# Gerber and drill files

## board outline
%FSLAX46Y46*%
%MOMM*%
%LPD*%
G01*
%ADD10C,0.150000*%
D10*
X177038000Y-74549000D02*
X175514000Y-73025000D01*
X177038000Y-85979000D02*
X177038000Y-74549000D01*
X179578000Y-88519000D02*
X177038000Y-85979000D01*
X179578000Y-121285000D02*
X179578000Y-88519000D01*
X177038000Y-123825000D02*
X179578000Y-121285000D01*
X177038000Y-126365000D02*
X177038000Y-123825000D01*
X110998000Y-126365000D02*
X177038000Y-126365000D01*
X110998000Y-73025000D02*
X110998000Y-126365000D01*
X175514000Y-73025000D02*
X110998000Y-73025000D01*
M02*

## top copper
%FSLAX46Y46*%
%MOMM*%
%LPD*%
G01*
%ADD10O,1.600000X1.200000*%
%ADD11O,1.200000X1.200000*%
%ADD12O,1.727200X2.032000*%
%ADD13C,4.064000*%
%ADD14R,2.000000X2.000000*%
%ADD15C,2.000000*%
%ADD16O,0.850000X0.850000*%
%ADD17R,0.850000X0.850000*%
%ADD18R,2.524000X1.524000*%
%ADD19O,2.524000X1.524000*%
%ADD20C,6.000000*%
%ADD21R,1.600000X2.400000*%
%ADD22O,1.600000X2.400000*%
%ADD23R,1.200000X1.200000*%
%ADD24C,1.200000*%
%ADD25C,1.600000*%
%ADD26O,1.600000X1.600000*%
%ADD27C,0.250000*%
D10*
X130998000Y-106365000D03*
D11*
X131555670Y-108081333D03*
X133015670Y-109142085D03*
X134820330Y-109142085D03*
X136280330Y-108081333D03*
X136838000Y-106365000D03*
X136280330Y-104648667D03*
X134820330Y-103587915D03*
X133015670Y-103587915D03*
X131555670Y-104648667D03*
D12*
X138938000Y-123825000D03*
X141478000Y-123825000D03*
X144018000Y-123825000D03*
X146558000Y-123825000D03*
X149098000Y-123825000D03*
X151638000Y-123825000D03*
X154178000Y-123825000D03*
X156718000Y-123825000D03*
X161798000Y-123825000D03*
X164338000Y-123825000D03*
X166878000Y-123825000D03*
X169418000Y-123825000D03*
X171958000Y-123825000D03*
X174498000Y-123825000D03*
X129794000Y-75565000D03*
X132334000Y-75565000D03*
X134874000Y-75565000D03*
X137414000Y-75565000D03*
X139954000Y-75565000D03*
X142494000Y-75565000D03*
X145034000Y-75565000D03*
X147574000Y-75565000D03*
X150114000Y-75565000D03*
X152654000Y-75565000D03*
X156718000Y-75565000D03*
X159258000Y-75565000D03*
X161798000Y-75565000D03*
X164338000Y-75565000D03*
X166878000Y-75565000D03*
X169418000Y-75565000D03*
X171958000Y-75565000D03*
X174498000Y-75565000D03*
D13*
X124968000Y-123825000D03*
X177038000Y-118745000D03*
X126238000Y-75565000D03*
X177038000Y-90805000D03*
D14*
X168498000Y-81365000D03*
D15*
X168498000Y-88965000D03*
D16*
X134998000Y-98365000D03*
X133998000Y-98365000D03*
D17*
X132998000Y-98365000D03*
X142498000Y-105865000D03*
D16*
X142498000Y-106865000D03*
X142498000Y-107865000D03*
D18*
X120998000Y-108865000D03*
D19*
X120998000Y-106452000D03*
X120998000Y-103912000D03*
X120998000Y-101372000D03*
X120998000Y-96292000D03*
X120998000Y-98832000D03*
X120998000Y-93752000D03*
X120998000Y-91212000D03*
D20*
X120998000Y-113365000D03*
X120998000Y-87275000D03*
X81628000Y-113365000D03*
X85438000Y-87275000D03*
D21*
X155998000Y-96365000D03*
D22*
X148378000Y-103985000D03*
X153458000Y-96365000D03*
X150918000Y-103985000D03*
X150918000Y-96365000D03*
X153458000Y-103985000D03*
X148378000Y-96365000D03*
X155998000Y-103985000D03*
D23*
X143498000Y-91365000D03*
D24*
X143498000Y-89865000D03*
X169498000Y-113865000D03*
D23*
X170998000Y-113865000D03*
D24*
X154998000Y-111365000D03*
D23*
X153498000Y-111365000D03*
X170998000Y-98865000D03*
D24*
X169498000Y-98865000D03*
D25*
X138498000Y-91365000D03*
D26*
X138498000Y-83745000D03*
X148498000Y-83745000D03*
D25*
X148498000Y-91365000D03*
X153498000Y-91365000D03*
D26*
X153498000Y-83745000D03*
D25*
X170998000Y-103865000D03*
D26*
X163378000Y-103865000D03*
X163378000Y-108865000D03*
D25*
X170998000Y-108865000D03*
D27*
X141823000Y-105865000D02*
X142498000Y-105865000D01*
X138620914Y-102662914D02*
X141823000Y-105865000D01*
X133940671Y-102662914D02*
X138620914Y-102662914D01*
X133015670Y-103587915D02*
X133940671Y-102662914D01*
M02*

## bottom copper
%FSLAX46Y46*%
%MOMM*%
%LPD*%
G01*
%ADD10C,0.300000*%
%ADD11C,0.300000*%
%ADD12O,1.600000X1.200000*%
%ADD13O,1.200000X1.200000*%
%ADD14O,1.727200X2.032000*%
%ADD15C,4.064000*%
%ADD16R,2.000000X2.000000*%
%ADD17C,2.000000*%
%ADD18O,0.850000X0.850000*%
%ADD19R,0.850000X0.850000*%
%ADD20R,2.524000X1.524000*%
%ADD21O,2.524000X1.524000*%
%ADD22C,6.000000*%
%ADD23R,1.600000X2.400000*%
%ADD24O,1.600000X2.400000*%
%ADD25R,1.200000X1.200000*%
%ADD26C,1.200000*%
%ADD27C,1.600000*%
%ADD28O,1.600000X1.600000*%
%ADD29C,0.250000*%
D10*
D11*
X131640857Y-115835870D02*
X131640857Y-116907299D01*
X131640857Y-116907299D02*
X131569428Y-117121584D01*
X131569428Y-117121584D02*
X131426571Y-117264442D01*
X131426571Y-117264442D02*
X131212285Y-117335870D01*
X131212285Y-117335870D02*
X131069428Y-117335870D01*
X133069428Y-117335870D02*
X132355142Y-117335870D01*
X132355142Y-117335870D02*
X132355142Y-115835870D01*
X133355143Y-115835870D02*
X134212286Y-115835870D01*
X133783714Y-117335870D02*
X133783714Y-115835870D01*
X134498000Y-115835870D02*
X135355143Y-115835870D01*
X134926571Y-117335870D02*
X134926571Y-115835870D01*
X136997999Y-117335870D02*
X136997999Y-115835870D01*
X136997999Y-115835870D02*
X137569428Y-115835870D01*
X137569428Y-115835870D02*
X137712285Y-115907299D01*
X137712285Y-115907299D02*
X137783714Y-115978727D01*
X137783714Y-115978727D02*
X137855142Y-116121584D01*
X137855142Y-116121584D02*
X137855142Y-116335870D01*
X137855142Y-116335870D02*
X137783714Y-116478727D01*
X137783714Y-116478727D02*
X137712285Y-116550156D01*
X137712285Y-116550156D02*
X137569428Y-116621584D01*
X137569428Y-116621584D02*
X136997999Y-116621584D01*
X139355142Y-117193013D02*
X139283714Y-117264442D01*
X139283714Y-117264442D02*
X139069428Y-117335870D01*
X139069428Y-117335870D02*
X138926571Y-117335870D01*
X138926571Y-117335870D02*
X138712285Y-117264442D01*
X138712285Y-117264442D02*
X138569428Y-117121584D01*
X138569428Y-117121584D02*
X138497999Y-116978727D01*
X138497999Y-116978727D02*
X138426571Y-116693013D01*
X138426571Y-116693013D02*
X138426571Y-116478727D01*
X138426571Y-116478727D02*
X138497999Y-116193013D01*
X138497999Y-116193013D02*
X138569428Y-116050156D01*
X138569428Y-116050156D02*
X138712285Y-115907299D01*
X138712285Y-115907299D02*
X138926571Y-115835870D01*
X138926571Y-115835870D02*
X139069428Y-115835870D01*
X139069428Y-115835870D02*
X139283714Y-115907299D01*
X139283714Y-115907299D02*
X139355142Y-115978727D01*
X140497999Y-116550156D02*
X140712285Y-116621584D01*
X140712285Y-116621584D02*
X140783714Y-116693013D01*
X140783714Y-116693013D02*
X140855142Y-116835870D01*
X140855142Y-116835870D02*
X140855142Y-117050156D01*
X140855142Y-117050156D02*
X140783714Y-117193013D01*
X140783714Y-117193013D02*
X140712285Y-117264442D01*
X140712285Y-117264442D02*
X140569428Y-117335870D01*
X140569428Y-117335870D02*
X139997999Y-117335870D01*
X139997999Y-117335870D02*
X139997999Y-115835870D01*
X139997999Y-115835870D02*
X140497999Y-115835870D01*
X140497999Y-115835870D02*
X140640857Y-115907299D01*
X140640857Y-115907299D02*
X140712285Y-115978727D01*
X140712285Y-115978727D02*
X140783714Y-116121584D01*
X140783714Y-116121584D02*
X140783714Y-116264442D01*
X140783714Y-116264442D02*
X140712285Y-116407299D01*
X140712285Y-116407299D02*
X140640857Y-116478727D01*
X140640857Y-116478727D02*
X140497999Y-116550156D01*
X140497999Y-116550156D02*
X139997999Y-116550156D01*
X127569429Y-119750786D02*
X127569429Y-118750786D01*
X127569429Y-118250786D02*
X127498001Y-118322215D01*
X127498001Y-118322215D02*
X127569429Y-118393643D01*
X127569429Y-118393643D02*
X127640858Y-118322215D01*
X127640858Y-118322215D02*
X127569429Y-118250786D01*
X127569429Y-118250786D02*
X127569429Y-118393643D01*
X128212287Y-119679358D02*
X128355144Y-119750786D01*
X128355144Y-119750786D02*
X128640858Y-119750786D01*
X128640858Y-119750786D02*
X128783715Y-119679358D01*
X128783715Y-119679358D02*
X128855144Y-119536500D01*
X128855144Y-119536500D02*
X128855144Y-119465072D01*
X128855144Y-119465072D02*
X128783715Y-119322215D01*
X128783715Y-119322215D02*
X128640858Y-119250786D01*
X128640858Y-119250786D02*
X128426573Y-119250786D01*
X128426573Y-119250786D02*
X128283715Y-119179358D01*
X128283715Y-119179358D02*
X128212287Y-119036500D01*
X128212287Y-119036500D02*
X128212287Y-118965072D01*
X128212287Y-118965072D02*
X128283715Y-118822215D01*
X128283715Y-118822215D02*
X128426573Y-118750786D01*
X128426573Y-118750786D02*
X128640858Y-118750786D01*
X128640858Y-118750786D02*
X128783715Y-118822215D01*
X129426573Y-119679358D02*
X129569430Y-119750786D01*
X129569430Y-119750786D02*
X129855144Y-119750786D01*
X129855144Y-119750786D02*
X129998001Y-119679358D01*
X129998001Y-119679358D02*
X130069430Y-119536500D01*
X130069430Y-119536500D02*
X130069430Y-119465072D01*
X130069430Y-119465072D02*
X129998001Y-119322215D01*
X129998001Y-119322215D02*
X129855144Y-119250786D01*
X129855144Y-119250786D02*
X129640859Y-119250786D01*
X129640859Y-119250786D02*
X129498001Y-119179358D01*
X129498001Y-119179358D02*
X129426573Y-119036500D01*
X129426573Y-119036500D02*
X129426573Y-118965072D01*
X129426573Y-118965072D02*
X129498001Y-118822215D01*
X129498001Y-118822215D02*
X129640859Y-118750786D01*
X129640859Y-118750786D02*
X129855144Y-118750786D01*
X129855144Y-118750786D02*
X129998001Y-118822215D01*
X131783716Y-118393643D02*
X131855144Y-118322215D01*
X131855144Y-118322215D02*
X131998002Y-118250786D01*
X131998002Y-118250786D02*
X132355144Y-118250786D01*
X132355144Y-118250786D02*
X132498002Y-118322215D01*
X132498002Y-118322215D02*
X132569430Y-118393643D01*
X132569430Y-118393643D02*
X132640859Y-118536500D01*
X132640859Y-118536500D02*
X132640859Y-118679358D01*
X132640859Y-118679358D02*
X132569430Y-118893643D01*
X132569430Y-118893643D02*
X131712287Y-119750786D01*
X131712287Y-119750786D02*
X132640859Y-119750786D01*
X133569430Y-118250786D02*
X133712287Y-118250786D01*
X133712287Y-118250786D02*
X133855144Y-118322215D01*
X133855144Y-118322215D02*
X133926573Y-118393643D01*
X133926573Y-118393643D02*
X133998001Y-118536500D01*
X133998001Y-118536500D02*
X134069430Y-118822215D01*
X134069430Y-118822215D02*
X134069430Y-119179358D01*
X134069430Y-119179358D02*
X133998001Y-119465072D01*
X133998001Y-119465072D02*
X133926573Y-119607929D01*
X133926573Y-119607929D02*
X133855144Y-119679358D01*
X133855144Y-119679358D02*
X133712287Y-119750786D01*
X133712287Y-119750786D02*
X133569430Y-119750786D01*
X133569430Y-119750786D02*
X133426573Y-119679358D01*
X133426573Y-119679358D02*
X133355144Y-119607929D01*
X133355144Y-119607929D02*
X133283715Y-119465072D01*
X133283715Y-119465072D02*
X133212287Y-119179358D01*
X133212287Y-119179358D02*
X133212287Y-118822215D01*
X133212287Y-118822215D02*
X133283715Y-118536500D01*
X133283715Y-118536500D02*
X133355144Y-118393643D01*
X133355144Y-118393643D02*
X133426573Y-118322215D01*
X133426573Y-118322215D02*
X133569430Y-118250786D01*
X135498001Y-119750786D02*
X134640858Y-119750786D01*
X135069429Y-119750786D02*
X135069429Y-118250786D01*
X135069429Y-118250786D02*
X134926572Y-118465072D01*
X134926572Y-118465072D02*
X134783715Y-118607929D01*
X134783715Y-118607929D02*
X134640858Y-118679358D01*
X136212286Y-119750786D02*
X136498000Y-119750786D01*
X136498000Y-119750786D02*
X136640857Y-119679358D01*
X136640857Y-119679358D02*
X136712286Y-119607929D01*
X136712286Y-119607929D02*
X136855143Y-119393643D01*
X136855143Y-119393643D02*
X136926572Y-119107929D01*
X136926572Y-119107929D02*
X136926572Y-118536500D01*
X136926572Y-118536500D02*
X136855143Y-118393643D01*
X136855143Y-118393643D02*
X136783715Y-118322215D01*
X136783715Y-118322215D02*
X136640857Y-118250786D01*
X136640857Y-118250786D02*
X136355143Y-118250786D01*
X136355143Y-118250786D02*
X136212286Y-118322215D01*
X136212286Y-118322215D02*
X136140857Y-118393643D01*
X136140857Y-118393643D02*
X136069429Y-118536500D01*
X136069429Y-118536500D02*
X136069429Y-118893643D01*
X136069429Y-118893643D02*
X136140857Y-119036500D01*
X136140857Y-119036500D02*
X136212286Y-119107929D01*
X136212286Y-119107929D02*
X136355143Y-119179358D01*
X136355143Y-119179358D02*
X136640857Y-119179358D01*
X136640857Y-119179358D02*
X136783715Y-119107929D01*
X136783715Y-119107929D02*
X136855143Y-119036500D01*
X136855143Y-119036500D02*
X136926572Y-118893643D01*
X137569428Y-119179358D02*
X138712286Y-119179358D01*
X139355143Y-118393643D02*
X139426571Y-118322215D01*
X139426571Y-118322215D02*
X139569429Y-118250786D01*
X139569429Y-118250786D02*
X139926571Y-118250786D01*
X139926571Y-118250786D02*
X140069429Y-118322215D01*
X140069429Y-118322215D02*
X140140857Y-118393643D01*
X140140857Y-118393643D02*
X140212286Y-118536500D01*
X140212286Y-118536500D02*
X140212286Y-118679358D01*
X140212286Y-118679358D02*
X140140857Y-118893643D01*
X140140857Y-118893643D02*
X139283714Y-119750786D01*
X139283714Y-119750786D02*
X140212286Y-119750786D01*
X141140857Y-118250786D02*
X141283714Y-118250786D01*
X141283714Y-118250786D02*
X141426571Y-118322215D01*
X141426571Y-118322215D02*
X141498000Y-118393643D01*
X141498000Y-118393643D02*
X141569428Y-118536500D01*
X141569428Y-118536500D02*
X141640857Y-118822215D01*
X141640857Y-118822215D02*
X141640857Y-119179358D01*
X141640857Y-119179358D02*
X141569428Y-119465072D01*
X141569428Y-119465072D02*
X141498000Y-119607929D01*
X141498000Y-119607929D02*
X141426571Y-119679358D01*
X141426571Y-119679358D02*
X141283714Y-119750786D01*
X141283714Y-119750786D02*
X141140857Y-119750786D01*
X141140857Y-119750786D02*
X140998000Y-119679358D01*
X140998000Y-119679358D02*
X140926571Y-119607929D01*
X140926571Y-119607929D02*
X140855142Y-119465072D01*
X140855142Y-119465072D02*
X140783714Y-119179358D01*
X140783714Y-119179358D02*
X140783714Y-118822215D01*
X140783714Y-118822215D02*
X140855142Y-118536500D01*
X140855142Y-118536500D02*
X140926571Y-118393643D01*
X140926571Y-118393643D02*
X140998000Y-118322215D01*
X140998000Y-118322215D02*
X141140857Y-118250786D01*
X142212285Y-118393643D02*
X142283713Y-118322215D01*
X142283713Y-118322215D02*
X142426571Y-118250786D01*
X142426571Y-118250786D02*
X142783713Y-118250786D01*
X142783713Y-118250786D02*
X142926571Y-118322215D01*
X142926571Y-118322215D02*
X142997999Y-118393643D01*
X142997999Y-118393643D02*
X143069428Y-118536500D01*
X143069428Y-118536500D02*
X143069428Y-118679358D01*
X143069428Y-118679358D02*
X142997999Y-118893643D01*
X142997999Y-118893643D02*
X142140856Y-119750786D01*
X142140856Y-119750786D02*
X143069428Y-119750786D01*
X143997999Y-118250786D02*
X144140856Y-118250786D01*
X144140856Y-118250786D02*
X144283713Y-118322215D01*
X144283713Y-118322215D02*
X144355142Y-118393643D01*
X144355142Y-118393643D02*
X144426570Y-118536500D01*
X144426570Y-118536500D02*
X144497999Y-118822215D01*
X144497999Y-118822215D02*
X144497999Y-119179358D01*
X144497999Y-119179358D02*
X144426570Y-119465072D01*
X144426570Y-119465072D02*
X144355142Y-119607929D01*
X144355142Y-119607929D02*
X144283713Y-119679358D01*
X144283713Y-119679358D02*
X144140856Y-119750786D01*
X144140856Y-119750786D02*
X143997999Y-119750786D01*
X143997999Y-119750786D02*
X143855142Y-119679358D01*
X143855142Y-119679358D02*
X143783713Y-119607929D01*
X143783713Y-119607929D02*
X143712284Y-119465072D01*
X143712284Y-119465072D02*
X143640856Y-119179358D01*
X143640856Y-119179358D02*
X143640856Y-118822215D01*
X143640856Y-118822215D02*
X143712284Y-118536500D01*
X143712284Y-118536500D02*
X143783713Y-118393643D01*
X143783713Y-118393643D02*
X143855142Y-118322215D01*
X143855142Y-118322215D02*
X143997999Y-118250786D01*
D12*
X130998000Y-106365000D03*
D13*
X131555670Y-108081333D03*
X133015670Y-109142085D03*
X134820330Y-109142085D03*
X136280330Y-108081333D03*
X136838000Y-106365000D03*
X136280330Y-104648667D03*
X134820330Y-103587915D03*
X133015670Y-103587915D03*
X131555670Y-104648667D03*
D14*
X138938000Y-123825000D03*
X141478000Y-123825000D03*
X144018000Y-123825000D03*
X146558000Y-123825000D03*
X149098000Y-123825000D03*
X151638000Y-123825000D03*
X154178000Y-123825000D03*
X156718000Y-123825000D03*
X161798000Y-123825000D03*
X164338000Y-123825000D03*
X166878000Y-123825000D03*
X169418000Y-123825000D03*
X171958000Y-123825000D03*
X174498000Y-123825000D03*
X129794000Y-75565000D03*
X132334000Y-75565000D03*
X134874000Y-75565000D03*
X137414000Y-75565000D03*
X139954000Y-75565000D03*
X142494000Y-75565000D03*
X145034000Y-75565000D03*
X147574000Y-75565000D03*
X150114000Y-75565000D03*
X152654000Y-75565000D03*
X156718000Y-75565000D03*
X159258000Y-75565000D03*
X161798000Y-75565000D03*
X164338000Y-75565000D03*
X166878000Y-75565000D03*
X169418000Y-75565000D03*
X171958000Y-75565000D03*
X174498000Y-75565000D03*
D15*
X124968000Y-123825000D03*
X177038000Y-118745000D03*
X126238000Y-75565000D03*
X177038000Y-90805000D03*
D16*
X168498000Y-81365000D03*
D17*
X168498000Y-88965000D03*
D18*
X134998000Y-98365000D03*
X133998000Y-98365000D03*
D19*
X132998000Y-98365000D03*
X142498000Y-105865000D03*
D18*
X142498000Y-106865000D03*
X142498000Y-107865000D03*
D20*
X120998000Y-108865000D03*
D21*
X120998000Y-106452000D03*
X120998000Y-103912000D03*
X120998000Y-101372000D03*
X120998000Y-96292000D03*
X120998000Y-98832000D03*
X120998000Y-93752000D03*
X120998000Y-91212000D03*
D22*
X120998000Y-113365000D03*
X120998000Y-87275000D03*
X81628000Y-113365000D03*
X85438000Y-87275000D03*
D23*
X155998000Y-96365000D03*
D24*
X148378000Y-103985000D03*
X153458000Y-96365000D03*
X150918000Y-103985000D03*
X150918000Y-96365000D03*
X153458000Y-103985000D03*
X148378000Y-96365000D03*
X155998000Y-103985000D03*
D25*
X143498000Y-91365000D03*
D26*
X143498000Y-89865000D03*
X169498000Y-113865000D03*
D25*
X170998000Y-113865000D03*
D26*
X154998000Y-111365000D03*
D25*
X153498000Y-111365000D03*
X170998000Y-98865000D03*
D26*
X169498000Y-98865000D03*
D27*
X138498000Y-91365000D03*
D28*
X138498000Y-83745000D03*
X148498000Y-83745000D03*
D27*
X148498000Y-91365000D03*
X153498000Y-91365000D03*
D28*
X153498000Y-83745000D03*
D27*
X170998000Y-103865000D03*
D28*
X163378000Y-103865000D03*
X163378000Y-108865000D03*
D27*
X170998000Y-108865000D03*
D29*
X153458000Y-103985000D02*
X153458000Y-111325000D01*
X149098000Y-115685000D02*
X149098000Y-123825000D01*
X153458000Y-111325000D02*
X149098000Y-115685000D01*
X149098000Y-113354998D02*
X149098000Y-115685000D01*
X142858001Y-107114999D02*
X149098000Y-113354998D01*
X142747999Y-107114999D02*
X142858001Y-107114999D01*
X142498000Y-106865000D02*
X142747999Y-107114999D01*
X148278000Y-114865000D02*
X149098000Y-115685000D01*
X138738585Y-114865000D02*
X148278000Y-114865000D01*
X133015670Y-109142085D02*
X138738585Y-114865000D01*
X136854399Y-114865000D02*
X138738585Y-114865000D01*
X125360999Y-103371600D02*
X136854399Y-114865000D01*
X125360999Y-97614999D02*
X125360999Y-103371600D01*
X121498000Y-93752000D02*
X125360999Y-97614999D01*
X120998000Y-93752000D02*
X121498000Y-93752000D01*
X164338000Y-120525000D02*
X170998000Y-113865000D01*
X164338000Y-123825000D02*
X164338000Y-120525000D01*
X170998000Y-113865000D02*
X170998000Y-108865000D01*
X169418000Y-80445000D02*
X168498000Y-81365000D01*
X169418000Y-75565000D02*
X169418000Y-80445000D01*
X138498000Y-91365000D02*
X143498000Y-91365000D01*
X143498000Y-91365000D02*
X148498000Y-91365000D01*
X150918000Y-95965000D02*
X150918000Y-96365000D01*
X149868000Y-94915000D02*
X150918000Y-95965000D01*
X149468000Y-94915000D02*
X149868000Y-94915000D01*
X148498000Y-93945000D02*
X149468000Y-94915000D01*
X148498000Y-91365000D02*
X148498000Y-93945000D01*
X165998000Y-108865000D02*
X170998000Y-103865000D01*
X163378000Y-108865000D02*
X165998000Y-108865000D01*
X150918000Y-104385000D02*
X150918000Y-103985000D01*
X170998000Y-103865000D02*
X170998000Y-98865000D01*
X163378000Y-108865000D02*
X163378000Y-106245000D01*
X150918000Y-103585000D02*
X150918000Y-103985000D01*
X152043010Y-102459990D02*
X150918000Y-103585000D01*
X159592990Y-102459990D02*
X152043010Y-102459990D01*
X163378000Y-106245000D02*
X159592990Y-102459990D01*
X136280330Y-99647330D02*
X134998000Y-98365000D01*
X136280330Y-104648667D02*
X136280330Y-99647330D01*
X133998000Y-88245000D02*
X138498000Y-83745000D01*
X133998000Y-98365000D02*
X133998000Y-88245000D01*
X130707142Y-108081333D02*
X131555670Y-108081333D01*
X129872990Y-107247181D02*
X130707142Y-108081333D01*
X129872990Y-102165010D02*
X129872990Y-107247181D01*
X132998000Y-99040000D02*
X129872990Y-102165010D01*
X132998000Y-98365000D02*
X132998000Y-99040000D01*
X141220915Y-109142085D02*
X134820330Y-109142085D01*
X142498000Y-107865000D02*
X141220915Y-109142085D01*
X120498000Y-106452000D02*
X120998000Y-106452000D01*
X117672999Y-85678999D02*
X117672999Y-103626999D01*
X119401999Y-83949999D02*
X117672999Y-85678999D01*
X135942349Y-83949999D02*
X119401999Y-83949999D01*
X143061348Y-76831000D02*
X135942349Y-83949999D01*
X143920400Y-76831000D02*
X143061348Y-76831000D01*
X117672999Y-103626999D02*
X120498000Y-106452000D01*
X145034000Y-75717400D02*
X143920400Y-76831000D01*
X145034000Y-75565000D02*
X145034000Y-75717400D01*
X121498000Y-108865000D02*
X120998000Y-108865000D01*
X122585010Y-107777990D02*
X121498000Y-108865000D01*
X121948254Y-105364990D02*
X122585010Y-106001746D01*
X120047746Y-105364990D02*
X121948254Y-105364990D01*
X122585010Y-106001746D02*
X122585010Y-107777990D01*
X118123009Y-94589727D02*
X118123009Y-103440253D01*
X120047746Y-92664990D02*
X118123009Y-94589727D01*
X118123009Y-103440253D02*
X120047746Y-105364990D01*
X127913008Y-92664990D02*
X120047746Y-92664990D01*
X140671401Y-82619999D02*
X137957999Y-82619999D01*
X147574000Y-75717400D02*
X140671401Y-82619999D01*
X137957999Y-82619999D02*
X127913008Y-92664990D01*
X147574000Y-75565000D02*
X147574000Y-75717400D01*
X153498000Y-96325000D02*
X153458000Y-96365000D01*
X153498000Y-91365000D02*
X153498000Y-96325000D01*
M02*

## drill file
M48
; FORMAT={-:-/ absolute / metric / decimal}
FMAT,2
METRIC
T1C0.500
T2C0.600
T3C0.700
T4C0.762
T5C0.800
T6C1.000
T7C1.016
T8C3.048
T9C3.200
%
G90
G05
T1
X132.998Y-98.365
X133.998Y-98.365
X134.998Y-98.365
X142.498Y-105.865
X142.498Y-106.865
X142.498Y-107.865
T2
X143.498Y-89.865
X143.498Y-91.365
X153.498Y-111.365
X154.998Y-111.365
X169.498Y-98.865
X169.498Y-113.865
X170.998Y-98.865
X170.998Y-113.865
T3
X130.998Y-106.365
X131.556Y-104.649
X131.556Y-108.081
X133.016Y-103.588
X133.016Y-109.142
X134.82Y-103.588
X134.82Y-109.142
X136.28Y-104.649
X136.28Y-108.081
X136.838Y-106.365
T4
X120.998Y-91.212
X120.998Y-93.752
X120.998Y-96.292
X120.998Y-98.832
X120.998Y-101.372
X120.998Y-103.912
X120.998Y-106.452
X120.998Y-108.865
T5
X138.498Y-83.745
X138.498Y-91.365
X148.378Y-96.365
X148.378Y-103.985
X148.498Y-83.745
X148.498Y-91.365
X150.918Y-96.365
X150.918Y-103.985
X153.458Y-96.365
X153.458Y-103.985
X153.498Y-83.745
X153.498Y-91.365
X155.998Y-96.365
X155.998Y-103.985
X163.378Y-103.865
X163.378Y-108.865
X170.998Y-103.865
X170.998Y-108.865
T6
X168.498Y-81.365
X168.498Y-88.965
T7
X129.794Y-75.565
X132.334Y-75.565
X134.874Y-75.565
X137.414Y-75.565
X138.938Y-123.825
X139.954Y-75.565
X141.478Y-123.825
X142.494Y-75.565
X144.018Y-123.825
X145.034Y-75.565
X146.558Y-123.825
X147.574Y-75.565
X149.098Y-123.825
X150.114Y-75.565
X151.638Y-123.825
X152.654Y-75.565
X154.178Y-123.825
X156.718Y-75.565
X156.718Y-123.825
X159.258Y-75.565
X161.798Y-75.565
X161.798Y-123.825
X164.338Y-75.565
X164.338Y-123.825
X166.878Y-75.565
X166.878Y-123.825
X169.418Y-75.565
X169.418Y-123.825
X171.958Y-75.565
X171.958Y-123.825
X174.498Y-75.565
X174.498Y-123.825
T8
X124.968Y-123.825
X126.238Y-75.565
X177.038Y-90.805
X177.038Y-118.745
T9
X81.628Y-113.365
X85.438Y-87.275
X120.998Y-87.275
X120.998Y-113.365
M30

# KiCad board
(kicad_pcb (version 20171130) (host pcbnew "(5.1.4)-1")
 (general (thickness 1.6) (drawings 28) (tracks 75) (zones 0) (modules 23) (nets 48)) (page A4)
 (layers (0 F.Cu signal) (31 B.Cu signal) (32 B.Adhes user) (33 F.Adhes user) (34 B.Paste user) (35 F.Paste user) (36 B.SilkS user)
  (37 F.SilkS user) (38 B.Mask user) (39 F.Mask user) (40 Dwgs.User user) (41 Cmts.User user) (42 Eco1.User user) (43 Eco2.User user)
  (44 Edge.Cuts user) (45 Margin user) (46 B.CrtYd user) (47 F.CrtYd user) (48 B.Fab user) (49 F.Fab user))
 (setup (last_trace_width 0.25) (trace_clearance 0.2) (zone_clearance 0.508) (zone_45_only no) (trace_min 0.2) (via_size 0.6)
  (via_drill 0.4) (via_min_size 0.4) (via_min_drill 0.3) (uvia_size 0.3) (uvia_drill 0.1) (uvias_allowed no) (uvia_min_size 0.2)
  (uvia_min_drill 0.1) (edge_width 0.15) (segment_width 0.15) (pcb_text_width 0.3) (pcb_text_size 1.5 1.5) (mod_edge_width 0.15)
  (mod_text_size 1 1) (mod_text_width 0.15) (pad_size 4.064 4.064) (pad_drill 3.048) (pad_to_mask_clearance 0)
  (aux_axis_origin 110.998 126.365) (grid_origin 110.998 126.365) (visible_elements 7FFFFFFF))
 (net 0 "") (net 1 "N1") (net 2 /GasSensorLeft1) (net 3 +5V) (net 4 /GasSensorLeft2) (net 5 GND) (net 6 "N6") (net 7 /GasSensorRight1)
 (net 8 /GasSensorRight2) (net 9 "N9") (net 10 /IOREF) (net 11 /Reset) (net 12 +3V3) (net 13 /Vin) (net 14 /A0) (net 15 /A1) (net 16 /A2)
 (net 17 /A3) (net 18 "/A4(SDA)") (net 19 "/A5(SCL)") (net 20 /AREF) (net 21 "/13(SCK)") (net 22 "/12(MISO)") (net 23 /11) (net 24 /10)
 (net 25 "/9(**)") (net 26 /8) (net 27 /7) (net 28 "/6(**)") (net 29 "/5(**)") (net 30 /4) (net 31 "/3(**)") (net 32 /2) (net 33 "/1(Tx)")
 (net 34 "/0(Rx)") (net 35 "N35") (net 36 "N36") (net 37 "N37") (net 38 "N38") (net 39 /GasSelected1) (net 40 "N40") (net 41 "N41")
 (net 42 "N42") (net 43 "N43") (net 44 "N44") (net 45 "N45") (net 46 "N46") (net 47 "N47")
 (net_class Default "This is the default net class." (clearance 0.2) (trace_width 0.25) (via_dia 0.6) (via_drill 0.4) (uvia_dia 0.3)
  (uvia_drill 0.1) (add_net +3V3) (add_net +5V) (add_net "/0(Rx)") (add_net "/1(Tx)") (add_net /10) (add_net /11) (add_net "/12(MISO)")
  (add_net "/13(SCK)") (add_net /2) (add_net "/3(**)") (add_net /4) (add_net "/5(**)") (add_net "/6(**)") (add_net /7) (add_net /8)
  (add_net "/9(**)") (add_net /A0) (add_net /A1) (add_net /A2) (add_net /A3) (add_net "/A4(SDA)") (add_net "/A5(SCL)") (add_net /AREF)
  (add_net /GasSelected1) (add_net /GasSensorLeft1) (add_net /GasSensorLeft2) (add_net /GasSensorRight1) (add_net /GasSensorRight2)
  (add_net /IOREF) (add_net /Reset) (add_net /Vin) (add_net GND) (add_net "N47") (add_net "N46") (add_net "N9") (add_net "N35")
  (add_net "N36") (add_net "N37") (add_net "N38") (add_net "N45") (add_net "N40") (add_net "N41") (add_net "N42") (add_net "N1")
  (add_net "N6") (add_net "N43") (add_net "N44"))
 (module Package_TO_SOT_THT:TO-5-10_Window (layer F.Cu) (at 130.998 106.365)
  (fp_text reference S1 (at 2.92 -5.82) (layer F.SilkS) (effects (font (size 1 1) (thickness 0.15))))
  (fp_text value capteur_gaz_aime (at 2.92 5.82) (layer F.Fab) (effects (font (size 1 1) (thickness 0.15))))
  (pad 1 thru_hole oval (at 0 0) (size 1.6 1.2) (drill 0.7) (layers *.Cu *.Mask) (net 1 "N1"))
  (pad 2 thru_hole oval (at 0.55767 1.716333) (size 1.2 1.2) (drill 0.7) (layers *.Cu *.Mask) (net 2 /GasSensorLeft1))
  (pad 3 thru_hole oval (at 2.01767 2.777085) (size 1.2 1.2) (drill 0.7) (layers *.Cu *.Mask) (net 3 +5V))
  (pad 4 thru_hole oval (at 3.82233 2.777085) (size 1.2 1.2) (drill 0.7) (layers *.Cu *.Mask) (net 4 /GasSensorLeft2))
  (pad 5 thru_hole oval (at 5.28233 1.716333) (size 1.2 1.2) (drill 0.7) (layers *.Cu *.Mask) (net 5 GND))
  (pad 6 thru_hole oval (at 5.84 0) (size 1.2 1.2) (drill 0.7) (layers *.Cu *.Mask) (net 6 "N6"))
  (pad 7 thru_hole oval (at 5.28233 -1.716333) (size 1.2 1.2) (drill 0.7) (layers *.Cu *.Mask) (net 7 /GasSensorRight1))
  (pad 8 thru_hole oval (at 3.82233 -2.777085) (size 1.2 1.2) (drill 0.7) (layers *.Cu *.Mask) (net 5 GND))
  (pad 9 thru_hole oval (at 2.01767 -2.777085) (size 1.2 1.2) (drill 0.7) (layers *.Cu *.Mask) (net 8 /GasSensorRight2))
  (pad 10 thru_hole oval (at 0.55767 -1.716333) (size 1.2 1.2) (drill 0.7) (layers *.Cu *.Mask) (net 5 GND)))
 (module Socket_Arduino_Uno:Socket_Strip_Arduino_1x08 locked (layer F.Cu) (at 138.938 123.825)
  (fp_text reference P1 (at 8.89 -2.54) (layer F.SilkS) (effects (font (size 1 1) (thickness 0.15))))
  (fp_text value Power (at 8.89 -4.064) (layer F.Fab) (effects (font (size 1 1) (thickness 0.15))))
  (pad 1 thru_hole oval (at 0 0) (size 1.7272 2.032) (drill 1.016) (layers *.Cu *.Mask F.SilkS) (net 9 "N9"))
  (pad 2 thru_hole oval (at 2.54 0) (size 1.7272 2.032) (drill 1.016) (layers *.Cu *.Mask F.SilkS) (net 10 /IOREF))
  (pad 3 thru_hole oval (at 5.08 0) (size 1.7272 2.032) (drill 1.016) (layers *.Cu *.Mask F.SilkS) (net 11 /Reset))
  (pad 4 thru_hole oval (at 7.62 0) (size 1.7272 2.032) (drill 1.016) (layers *.Cu *.Mask F.SilkS) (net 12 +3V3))
  (pad 5 thru_hole oval (at 10.16 0) (size 1.7272 2.032) (drill 1.016) (layers *.Cu *.Mask F.SilkS) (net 3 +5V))
  (pad 6 thru_hole oval (at 12.7 0) (size 1.7272 2.032) (drill 1.016) (layers *.Cu *.Mask F.SilkS) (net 5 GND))
  (pad 7 thru_hole oval (at 15.24 0) (size 1.7272 2.032) (drill 1.016) (layers *.Cu *.Mask F.SilkS) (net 5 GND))
  (pad 8 thru_hole oval (at 17.78 0) (size 1.7272 2.032) (drill 1.016) (layers *.Cu *.Mask F.SilkS) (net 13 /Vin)))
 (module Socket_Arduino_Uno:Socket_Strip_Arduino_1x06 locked (layer F.Cu) (at 161.798 123.825)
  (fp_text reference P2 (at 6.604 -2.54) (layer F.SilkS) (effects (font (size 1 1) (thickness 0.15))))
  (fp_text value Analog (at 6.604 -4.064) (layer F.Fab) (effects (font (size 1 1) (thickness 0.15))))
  (pad 1 thru_hole oval (at 0 0) (size 1.7272 2.032) (drill 1.016) (layers *.Cu *.Mask F.SilkS) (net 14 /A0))
  (pad 2 thru_hole oval (at 2.54 0) (size 1.7272 2.032) (drill 1.016) (layers *.Cu *.Mask F.SilkS) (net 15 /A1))
  (pad 3 thru_hole oval (at 5.08 0) (size 1.7272 2.032) (drill 1.016) (layers *.Cu *.Mask F.SilkS) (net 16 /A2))
  (pad 4 thru_hole oval (at 7.62 0) (size 1.7272 2.032) (drill 1.016) (layers *.Cu *.Mask F.SilkS) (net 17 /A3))
  (pad 5 thru_hole oval (at 10.16 0) (size 1.7272 2.032) (drill 1.016) (layers *.Cu *.Mask F.SilkS) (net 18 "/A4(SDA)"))
  (pad 6 thru_hole oval (at 12.7 0) (size 1.7272 2.032) (drill 1.016) (layers *.Cu *.Mask F.SilkS) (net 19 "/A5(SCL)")))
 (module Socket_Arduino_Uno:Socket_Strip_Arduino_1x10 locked (layer F.Cu) (at 129.794 75.565)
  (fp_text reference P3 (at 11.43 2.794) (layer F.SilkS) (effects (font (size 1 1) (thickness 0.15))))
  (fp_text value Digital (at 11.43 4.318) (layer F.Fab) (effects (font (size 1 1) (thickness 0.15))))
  (pad 1 thru_hole oval (at 0 0) (size 1.7272 2.032) (drill 1.016) (layers *.Cu *.Mask F.SilkS) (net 19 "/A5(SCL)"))
  (pad 2 thru_hole oval (at 2.54 0) (size 1.7272 2.032) (drill 1.016) (layers *.Cu *.Mask F.SilkS) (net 18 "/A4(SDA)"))
  (pad 3 thru_hole oval (at 5.08 0) (size 1.7272 2.032) (drill 1.016) (layers *.Cu *.Mask F.SilkS) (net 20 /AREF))
  (pad 4 thru_hole oval (at 7.62 0) (size 1.7272 2.032) (drill 1.016) (layers *.Cu *.Mask F.SilkS) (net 5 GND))
  (pad 5 thru_hole oval (at 10.16 0) (size 1.7272 2.032) (drill 1.016) (layers *.Cu *.Mask F.SilkS) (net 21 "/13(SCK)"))
  (pad 6 thru_hole oval (at 12.7 0) (size 1.7272 2.032) (drill 1.016) (layers *.Cu *.Mask F.SilkS) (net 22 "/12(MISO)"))
  (pad 7 thru_hole oval (at 15.24 0) (size 1.7272 2.032) (drill 1.016) (layers *.Cu *.Mask F.SilkS) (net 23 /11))
  (pad 8 thru_hole oval (at 17.78 0) (size 1.7272 2.032) (drill 1.016) (layers *.Cu *.Mask F.SilkS) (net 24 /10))
  (pad 9 thru_hole oval (at 20.32 0) (size 1.7272 2.032) (drill 1.016) (layers *.Cu *.Mask F.SilkS) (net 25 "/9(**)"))
  (pad 10 thru_hole oval (at 22.86 0) (size 1.7272 2.032) (drill 1.016) (layers *.Cu *.Mask F.SilkS) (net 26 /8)))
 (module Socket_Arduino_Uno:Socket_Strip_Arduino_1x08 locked (layer F.Cu) (at 156.718 75.565)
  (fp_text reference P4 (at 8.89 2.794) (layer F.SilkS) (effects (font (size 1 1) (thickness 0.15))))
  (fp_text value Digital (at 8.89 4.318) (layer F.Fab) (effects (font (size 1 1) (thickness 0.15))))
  (pad 1 thru_hole oval (at 0 0) (size 1.7272 2.032) (drill 1.016) (layers *.Cu *.Mask F.SilkS) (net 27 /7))
  (pad 2 thru_hole oval (at 2.54 0) (size 1.7272 2.032) (drill 1.016) (layers *.Cu *.Mask F.SilkS) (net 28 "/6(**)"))
  (pad 3 thru_hole oval (at 5.08 0) (size 1.7272 2.032) (drill 1.016) (layers *.Cu *.Mask F.SilkS) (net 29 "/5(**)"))
  (pad 4 thru_hole oval (at 7.62 0) (size 1.7272 2.032) (drill 1.016) (layers *.Cu *.Mask F.SilkS) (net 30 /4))
  (pad 5 thru_hole oval (at 10.16 0) (size 1.7272 2.032) (drill 1.016) (layers *.Cu *.Mask F.SilkS) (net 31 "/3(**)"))
  (pad 6 thru_hole oval (at 12.7 0) (size 1.7272 2.032) (drill 1.016) (layers *.Cu *.Mask F.SilkS) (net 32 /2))
  (pad 7 thru_hole oval (at 15.24 0) (size 1.7272 2.032) (drill 1.016) (layers *.Cu *.Mask F.SilkS) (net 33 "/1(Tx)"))
  (pad 8 thru_hole oval (at 17.78 0) (size 1.7272 2.032) (drill 1.016) (layers *.Cu *.Mask F.SilkS) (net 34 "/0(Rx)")))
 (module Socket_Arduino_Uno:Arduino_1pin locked (layer F.Cu) (at 124.968 123.825)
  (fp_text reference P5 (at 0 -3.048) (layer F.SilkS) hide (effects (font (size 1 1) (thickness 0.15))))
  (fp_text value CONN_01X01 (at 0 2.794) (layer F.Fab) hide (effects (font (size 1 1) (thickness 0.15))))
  (pad 1 thru_hole circle (at 0 0) (size 4.064 4.064) (drill 3.048) (layers *.Cu *.Mask F.SilkS) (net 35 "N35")))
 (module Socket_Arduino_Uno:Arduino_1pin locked (layer F.Cu) (at 177.038 118.745)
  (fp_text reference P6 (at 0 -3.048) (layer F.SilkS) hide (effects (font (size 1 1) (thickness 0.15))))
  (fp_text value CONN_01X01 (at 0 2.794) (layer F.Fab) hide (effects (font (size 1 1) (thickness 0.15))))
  (pad 1 thru_hole circle (at 0 0) (size 4.064 4.064) (drill 3.048) (layers *.Cu *.Mask F.SilkS) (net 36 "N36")))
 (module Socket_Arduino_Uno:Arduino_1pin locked (layer F.Cu) (at 126.238 75.565)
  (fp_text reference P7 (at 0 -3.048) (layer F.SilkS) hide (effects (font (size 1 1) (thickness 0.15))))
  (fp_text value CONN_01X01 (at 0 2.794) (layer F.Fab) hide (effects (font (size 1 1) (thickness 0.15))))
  (pad 1 thru_hole circle (at 0 0) (size 4.064 4.064) (drill 3.048) (layers *.Cu *.Mask F.SilkS) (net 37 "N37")))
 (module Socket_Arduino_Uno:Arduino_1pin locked (layer F.Cu) (at 177.038 90.805)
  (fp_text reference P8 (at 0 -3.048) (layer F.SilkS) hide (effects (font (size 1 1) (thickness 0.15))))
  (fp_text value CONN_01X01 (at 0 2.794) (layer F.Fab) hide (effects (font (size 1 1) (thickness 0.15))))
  (pad 1 thru_hole circle (at 0 0) (size 4.064 4.064) (drill 3.048) (layers *.Cu *.Mask F.SilkS) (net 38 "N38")))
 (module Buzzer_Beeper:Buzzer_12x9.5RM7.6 (layer F.Cu) (at 168.498 81.365 270)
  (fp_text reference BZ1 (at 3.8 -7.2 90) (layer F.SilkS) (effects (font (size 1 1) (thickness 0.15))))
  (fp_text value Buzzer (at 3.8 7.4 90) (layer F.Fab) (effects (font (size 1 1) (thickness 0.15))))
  (pad 1 thru_hole rect (at 0 0 270) (size 2 2) (drill 1) (layers *.Cu *.Mask) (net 32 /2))
  (pad 2 thru_hole circle (at 7.6 0 270) (size 2 2) (drill 1) (layers *.Cu *.Mask) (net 5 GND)))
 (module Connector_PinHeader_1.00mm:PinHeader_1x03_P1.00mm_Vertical (layer F.Cu) (at 132.998 98.365 90)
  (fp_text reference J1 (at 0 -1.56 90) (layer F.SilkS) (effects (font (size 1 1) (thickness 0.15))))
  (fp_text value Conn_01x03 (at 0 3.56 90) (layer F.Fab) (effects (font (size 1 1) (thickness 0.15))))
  (pad 3 thru_hole oval (at 0 2 90) (size 0.85 0.85) (drill 0.5) (layers *.Cu *.Mask) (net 7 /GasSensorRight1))
  (pad 2 thru_hole oval (at 0 1 90) (size 0.85 0.85) (drill 0.5) (layers *.Cu *.Mask) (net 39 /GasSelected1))
  (pad 1 thru_hole rect (at 0 0 90) (size 0.85 0.85) (drill 0.5) (layers *.Cu *.Mask) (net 2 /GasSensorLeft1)))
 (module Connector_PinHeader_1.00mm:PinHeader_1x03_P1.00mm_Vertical (layer F.Cu) (at 142.498 105.865)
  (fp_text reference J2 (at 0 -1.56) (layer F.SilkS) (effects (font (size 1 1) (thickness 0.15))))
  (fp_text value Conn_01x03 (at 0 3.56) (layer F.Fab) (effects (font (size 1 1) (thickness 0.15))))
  (pad 1 thru_hole rect (at 0 0) (size 0.85 0.85) (drill 0.5) (layers *.Cu *.Mask) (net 8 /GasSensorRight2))
  (pad 2 thru_hole oval (at 0 1) (size 0.85 0.85) (drill 0.5) (layers *.Cu *.Mask) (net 3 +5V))
  (pad 3 thru_hole oval (at 0 2) (size 0.85 0.85) (drill 0.5) (layers *.Cu *.Mask) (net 4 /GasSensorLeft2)))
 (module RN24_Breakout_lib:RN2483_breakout (layer F.Cu) (at 120.998 108.865 90)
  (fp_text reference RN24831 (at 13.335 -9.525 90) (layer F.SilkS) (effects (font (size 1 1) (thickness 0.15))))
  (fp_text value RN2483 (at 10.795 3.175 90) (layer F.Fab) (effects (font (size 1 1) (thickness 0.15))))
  (pad 1 thru_hole rect (at 0 0 90) (size 1.524 2.524) (drill 0.762) (layers *.Cu *.Mask) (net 24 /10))
  (pad 2 thru_hole oval (at 2.413 0 90) (size 1.524 2.524) (drill 0.762) (layers *.Cu *.Mask) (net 23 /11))
  (pad 3 thru_hole oval (at 4.953 0 90) (size 1.524 2.524) (drill 0.762) (layers *.Cu *.Mask) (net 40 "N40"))
  (pad 4 thru_hole oval (at 7.493 0 90) (size 1.524 2.524) (drill 0.762) (layers *.Cu *.Mask) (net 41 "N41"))
  (pad 6 thru_hole oval (at 12.573 0 90) (size 1.524 2.524) (drill 0.762) (layers *.Cu *.Mask))
  (pad 5 thru_hole oval (at 10.033 0 90) (size 1.524 2.524) (drill 0.762) (layers *.Cu *.Mask) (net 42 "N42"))
  (pad 7 thru_hole oval (at 15.113 0 90) (size 1.524 2.524) (drill 0.762) (layers *.Cu *.Mask) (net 3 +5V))
  (pad 8 thru_hole oval (at 17.653 0 90) (size 1.524 2.524) (drill 0.762) (layers *.Cu *.Mask) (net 5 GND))
  (pad "" np_thru_hole circle (at -4.5 0 90) (size 6 6) (drill 3.2) (layers *.Cu *.Mask))
  (pad "" np_thru_hole circle (at 21.59 0 90) (size 6 6) (drill 3.2) (layers *.Cu *.Mask))
  (pad "" np_thru_hole circle (at -4.5 -39.37 90) (size 6 6) (drill 3.2) (layers *.Cu *.Mask))
  (pad "" np_thru_hole circle (at 21.59 -35.56 90) (size 6 6) (drill 3.2) (layers *.Cu *.Mask)))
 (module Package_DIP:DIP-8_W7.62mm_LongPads (layer F.Cu) (at 155.998 96.365 270)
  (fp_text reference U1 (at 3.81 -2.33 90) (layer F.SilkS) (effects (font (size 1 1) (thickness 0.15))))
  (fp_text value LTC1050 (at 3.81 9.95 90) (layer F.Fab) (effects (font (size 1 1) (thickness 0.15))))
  (pad 1 thru_hole rect (at 0 0 270) (size 2.4 1.6) (drill 0.8) (layers *.Cu *.Mask) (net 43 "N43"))
  (pad 5 thru_hole oval (at 7.62 7.62 270) (size 2.4 1.6) (drill 0.8) (layers *.Cu *.Mask) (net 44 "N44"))
  (pad 2 thru_hole oval (at 0 2.54 270) (size 2.4 1.6) (drill 0.8) (layers *.Cu *.Mask) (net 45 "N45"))
  (pad 6 thru_hole oval (at 7.62 5.08 270) (size 2.4 1.6) (drill 0.8) (layers *.Cu *.Mask) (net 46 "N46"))
  (pad 3 thru_hole oval (at 0 5.08 270) (size 2.4 1.6) (drill 0.8) (layers *.Cu *.Mask) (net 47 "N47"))
  (pad 7 thru_hole oval (at 7.62 2.54 270) (size 2.4 1.6) (drill 0.8) (layers *.Cu *.Mask) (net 3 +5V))
  (pad 4 thru_hole oval (at 0 7.62 270) (size 2.4 1.6) (drill 0.8) (layers *.Cu *.Mask) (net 5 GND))
  (pad 8 thru_hole oval (at 7.62 0 270) (size 2.4 1.6) (drill 0.8) (layers *.Cu *.Mask)))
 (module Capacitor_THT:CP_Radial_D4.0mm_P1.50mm (layer F.Cu) (at 143.498 91.365 90)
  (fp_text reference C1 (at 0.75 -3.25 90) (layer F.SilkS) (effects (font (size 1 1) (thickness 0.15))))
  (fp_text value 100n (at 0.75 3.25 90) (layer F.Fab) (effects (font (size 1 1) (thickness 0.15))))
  (pad 1 thru_hole rect (at 0 0 90) (size 1.2 1.2) (drill 0.6) (layers *.Cu *.Mask) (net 47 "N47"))
  (pad 2 thru_hole circle (at 1.5 0 90) (size 1.2 1.2) (drill 0.6) (layers *.Cu *.Mask) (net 5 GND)))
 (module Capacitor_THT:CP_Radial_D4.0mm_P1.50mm (layer F.Cu) (at 170.998 113.865 180)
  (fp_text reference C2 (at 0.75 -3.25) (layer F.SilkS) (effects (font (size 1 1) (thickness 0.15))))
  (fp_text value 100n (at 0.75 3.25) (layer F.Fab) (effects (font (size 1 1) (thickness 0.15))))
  (pad 2 thru_hole circle (at 1.5 0 180) (size 1.2 1.2) (drill 0.6) (layers *.Cu *.Mask) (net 5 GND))
  (pad 1 thru_hole rect (at 0 0 180) (size 1.2 1.2) (drill 0.6) (layers *.Cu *.Mask) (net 15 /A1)))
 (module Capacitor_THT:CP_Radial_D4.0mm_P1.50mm (layer F.Cu) (at 153.498 111.365)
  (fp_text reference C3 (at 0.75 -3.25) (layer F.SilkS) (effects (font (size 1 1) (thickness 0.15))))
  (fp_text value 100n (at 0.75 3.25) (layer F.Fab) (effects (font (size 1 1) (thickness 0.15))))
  (pad 2 thru_hole circle (at 1.5 0) (size 1.2 1.2) (drill 0.6) (layers *.Cu *.Mask) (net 5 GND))
  (pad 1 thru_hole rect (at 0 0) (size 1.2 1.2) (drill 0.6) (layers *.Cu *.Mask) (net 3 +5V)))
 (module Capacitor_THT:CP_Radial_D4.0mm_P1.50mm (layer F.Cu) (at 170.998 98.865 180)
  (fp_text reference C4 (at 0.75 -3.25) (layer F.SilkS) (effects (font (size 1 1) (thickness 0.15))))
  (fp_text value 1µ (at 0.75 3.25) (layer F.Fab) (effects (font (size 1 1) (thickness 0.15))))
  (pad 1 thru_hole rect (at 0 0 180) (size 1.2 1.2) (drill 0.6) (layers *.Cu *.Mask) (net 46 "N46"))
  (pad 2 thru_hole circle (at 1.5 0 180) (size 1.2 1.2) (drill 0.6) (layers *.Cu *.Mask) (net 5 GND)))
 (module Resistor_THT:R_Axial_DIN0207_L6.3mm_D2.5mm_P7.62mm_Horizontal (layer F.Cu) (at 138.498 91.365 90)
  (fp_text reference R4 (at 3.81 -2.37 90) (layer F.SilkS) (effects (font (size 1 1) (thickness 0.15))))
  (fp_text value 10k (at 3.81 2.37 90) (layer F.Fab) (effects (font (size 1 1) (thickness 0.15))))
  (pad 1 thru_hole circle (at 0 0 90) (size 1.6 1.6) (drill 0.8) (layers *.Cu *.Mask) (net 47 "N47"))
  (pad 2 thru_hole oval (at 7.62 0 90) (size 1.6 1.6) (drill 0.8) (layers *.Cu *.Mask) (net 39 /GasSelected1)))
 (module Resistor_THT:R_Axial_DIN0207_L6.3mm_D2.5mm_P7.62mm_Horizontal (layer F.Cu) (at 148.498 91.365 90)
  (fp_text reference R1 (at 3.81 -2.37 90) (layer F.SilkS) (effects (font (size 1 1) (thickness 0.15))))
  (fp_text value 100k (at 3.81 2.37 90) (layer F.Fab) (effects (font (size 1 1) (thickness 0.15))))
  (pad 2 thru_hole oval (at 7.62 0 90) (size 1.6 1.6) (drill 0.8) (layers *.Cu *.Mask) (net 5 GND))
  (pad 1 thru_hole circle (at 0 0 90) (size 1.6 1.6) (drill 0.8) (layers *.Cu *.Mask) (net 47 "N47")))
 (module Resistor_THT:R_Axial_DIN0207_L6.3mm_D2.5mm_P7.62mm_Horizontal (layer F.Cu) (at 153.498 91.365 90)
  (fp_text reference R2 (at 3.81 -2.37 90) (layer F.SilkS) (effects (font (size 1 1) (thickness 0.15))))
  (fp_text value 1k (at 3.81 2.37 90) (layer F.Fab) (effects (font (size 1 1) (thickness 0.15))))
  (pad 1 thru_hole circle (at 0 0 90) (size 1.6 1.6) (drill 0.8) (layers *.Cu *.Mask) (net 45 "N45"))
  (pad 2 thru_hole oval (at 7.62 0 90) (size 1.6 1.6) (drill 0.8) (layers *.Cu *.Mask) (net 5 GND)))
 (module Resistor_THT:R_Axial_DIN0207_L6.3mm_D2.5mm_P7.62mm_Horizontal (layer F.Cu) (at 170.998 103.865 180)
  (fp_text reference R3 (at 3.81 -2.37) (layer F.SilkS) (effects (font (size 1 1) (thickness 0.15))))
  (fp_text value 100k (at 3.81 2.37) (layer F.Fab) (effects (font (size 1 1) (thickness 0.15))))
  (pad 1 thru_hole circle (at 0 0 180) (size 1.6 1.6) (drill 0.8) (layers *.Cu *.Mask) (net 46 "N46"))
  (pad 2 thru_hole oval (at 7.62 0 180) (size 1.6 1.6) (drill 0.8) (layers *.Cu *.Mask) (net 5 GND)))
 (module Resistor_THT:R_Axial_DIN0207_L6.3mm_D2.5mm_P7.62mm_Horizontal (layer F.Cu) (at 170.998 108.865 180)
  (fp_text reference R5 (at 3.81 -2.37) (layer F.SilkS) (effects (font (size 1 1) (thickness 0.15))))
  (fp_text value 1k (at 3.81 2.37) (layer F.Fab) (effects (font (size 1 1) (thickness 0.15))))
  (pad 2 thru_hole oval (at 7.62 0 180) (size 1.6 1.6) (drill 0.8) (layers *.Cu *.Mask) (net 46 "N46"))
  (pad 1 thru_hole circle (at 0 0 180) (size 1.6 1.6) (drill 0.8) (layers *.Cu *.Mask) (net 15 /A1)))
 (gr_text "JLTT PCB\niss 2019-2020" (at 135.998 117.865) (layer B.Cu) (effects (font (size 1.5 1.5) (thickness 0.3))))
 (gr_line (start 177.038 74.549) (end 175.514 73.025) (angle 90) (layer Edge.Cuts) (width 0.15))
 (gr_line (start 177.038 85.979) (end 177.038 74.549) (angle 90) (layer Edge.Cuts) (width 0.15))
 (gr_line (start 179.578 88.519) (end 177.038 85.979) (angle 90) (layer Edge.Cuts) (width 0.15))
 (gr_line (start 179.578 121.285) (end 179.578 88.519) (angle 90) (layer Edge.Cuts) (width 0.15))
 (gr_line (start 177.038 123.825) (end 179.578 121.285) (angle 90) (layer Edge.Cuts) (width 0.15))
 (gr_line (start 177.038 126.365) (end 177.038 123.825) (angle 90) (layer Edge.Cuts) (width 0.15))
 (gr_line (start 110.998 126.365) (end 177.038 126.365) (angle 90) (layer Edge.Cuts) (width 0.15))
 (gr_line (start 110.998 73.025) (end 110.998 126.365) (angle 90) (layer Edge.Cuts) (width 0.15))
 (gr_line (start 175.514 73.025) (end 110.998 73.025) (angle 90) (layer Edge.Cuts) (width 0.15))
 (segment (start 153.458 103.985) (end 153.458 111.325) (width 0.25) (layer B.Cu) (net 3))
 (segment (start 149.098 115.685) (end 149.098 123.825) (width 0.25) (layer B.Cu) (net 3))
 (segment (start 153.458 111.325) (end 149.098 115.685) (width 0.25) (layer B.Cu) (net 3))
 (segment (start 149.098 113.354998) (end 149.098 115.685) (width 0.25) (layer B.Cu) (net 3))
 (segment (start 142.858001 107.114999) (end 149.098 113.354998) (width 0.25) (layer B.Cu) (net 3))
 (segment (start 142.747999 107.114999) (end 142.858001 107.114999) (width 0.25) (layer B.Cu) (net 3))
 (segment (start 142.498 106.865) (end 142.747999 107.114999) (width 0.25) (layer B.Cu) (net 3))
 (segment (start 148.278 114.865) (end 149.098 115.685) (width 0.25) (layer B.Cu) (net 3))
 (segment (start 138.738585 114.865) (end 148.278 114.865) (width 0.25) (layer B.Cu) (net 3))
 (segment (start 133.01567 109.142085) (end 138.738585 114.865) (width 0.25) (layer B.Cu) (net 3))
 (segment (start 136.854399 114.865) (end 138.738585 114.865) (width 0.25) (layer B.Cu) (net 3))
 (segment (start 125.360999 103.3716) (end 136.854399 114.865) (width 0.25) (layer B.Cu) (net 3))
 (segment (start 125.360999 97.614999) (end 125.360999 103.3716) (width 0.25) (layer B.Cu) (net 3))
 (segment (start 121.498 93.752) (end 125.360999 97.614999) (width 0.25) (layer B.Cu) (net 3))
 (segment (start 120.998 93.752) (end 121.498 93.752) (width 0.25) (layer B.Cu) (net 3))
 (segment (start 164.338 120.525) (end 170.998 113.865) (width 0.25) (layer B.Cu) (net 15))
 (segment (start 164.338 123.825) (end 164.338 120.525) (width 0.25) (layer B.Cu) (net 15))
 (segment (start 170.998 113.865) (end 170.998 108.865) (width 0.25) (layer B.Cu) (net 15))
 (segment (start 169.418 80.445) (end 168.498 81.365) (width 0.25) (layer B.Cu) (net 32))
 (segment (start 169.418 75.565) (end 169.418 80.445) (width 0.25) (layer B.Cu) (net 32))
 (segment (start 138.498 91.365) (end 143.498 91.365) (width 0.25) (layer B.Cu) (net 47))
 (segment (start 143.498 91.365) (end 148.498 91.365) (width 0.25) (layer B.Cu) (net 47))
 (segment (start 150.918 95.965) (end 150.918 96.365) (width 0.25) (layer B.Cu) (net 47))
 (segment (start 149.868 94.915) (end 150.918 95.965) (width 0.25) (layer B.Cu) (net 47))
 (segment (start 149.468 94.915) (end 149.868 94.915) (width 0.25) (layer B.Cu) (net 47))
 (segment (start 148.498 93.945) (end 149.468 94.915) (width 0.25) (layer B.Cu) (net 47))
 (segment (start 148.498 91.365) (end 148.498 93.945) (width 0.25) (layer B.Cu) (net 47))
 (segment (start 165.998 108.865) (end 170.998 103.865) (width 0.25) (layer B.Cu) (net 46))
 (segment (start 163.378 108.865) (end 165.998 108.865) (width 0.25) (layer B.Cu) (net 46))
 (segment (start 150.918 104.385) (end 150.918 103.985) (width 0.25) (layer B.Cu) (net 46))
 (segment (start 170.998 103.865) (end 170.998 98.865) (width 0.25) (layer B.Cu) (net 46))
 (segment (start 163.378 108.865) (end 163.378 106.245) (width 0.25) (layer B.Cu) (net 46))
 (segment (start 150.918 103.585) (end 150.918 103.985) (width 0.25) (layer B.Cu) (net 46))
 (segment (start 152.04301 102.45999) (end 150.918 103.585) (width 0.25) (layer B.Cu) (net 46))
 (segment (start 159.59299 102.45999) (end 152.04301 102.45999) (width 0.25) (layer B.Cu) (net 46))
 (segment (start 163.378 106.245) (end 159.59299 102.45999) (width 0.25) (layer B.Cu) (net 46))
 (segment (start 136.28033 99.64733) (end 134.998 98.365) (width 0.25) (layer B.Cu) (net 7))
 (segment (start 136.28033 104.648667) (end 136.28033 99.64733) (width 0.25) (layer B.Cu) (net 7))
 (segment (start 133.998 88.245) (end 138.498 83.745) (width 0.25) (layer B.Cu) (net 39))
 (segment (start 133.998 98.365) (end 133.998 88.245) (width 0.25) (layer B.Cu) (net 39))
 (segment (start 130.707142 108.081333) (end 131.55567 108.081333) (width 0.25) (layer B.Cu) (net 2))
 (segment (start 129.87299 107.247181) (end 130.707142 108.081333) (width 0.25) (layer B.Cu) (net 2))
 (segment (start 129.87299 102.16501) (end 129.87299 107.247181) (width 0.25) (layer B.Cu) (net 2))
 (segment (start 132.998 99.04) (end 129.87299 102.16501) (width 0.25) (layer B.Cu) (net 2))
 (segment (start 132.998 98.365) (end 132.998 99.04) (width 0.25) (layer B.Cu) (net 2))
 (segment (start 141.823 105.865) (end 142.498 105.865) (width 0.25) (layer F.Cu) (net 8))
 (segment (start 138.620914 102.662914) (end 141.823 105.865) (width 0.25) (layer F.Cu) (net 8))
 (segment (start 133.940671 102.662914) (end 138.620914 102.662914) (width 0.25) (layer F.Cu) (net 8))
 (segment (start 133.01567 103.587915) (end 133.940671 102.662914) (width 0.25) (layer F.Cu) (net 8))
 (segment (start 141.220915 109.142085) (end 134.82033 109.142085) (width 0.25) (layer B.Cu) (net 4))
 (segment (start 142.498 107.865) (end 141.220915 109.142085) (width 0.25) (layer B.Cu) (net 4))
 (segment (start 120.498 106.452) (end 120.998 106.452) (width 0.25) (layer B.Cu) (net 23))
 (segment (start 117.672999 85.678999) (end 117.672999 103.626999) (width 0.25) (layer B.Cu) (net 23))
 (segment (start 119.401999 83.949999) (end 117.672999 85.678999) (width 0.25) (layer B.Cu) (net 23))
 (segment (start 135.942349 83.949999) (end 119.401999 83.949999) (width 0.25) (layer B.Cu) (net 23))
 (segment (start 143.061348 76.831) (end 135.942349 83.949999) (width 0.25) (layer B.Cu) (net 23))
 (segment (start 143.9204 76.831) (end 143.061348 76.831) (width 0.25) (layer B.Cu) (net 23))
 (segment (start 117.672999 103.626999) (end 120.498 106.452) (width 0.25) (layer B.Cu) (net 23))
 (segment (start 145.034 75.7174) (end 143.9204 76.831) (width 0.25) (layer B.Cu) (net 23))
 (segment (start 145.034 75.565) (end 145.034 75.7174) (width 0.25) (layer B.Cu) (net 23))
 (segment (start 121.498 108.865) (end 120.998 108.865) (width 0.25) (layer B.Cu) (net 24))
 (segment (start 122.58501 107.77799) (end 121.498 108.865) (width 0.25) (layer B.Cu) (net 24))
 (segment (start 121.948254 105.36499) (end 122.58501 106.001746) (width 0.25) (layer B.Cu) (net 24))
 (segment (start 120.047746 105.36499) (end 121.948254 105.36499) (width 0.25) (layer B.Cu) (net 24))
 (segment (start 122.58501 106.001746) (end 122.58501 107.77799) (width 0.25) (layer B.Cu) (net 24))
 (segment (start 118.123009 94.589727) (end 118.123009 103.440253) (width 0.25) (layer B.Cu) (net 24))
 (segment (start 120.047746 92.66499) (end 118.123009 94.589727) (width 0.25) (layer B.Cu) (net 24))
 (segment (start 118.123009 103.440253) (end 120.047746 105.36499) (width 0.25) (layer B.Cu) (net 24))
 (segment (start 127.913008 92.66499) (end 120.047746 92.66499) (width 0.25) (layer B.Cu) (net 24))
 (segment (start 140.671401 82.619999) (end 137.957999 82.619999) (width 0.25) (layer B.Cu) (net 24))
 (segment (start 147.574 75.7174) (end 140.671401 82.619999) (width 0.25) (layer B.Cu) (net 24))
 (segment (start 137.957999 82.619999) (end 127.913008 92.66499) (width 0.25) (layer B.Cu) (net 24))
 (segment (start 147.574 75.565) (end 147.574 75.7174) (width 0.25) (layer B.Cu) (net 24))
 (segment (start 153.498 96.325) (end 153.458 96.365) (width 0.25) (layer B.Cu) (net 45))
 (segment (start 153.498 91.365) (end 153.498 96.325) (width 0.25) (layer B.Cu) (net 45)))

